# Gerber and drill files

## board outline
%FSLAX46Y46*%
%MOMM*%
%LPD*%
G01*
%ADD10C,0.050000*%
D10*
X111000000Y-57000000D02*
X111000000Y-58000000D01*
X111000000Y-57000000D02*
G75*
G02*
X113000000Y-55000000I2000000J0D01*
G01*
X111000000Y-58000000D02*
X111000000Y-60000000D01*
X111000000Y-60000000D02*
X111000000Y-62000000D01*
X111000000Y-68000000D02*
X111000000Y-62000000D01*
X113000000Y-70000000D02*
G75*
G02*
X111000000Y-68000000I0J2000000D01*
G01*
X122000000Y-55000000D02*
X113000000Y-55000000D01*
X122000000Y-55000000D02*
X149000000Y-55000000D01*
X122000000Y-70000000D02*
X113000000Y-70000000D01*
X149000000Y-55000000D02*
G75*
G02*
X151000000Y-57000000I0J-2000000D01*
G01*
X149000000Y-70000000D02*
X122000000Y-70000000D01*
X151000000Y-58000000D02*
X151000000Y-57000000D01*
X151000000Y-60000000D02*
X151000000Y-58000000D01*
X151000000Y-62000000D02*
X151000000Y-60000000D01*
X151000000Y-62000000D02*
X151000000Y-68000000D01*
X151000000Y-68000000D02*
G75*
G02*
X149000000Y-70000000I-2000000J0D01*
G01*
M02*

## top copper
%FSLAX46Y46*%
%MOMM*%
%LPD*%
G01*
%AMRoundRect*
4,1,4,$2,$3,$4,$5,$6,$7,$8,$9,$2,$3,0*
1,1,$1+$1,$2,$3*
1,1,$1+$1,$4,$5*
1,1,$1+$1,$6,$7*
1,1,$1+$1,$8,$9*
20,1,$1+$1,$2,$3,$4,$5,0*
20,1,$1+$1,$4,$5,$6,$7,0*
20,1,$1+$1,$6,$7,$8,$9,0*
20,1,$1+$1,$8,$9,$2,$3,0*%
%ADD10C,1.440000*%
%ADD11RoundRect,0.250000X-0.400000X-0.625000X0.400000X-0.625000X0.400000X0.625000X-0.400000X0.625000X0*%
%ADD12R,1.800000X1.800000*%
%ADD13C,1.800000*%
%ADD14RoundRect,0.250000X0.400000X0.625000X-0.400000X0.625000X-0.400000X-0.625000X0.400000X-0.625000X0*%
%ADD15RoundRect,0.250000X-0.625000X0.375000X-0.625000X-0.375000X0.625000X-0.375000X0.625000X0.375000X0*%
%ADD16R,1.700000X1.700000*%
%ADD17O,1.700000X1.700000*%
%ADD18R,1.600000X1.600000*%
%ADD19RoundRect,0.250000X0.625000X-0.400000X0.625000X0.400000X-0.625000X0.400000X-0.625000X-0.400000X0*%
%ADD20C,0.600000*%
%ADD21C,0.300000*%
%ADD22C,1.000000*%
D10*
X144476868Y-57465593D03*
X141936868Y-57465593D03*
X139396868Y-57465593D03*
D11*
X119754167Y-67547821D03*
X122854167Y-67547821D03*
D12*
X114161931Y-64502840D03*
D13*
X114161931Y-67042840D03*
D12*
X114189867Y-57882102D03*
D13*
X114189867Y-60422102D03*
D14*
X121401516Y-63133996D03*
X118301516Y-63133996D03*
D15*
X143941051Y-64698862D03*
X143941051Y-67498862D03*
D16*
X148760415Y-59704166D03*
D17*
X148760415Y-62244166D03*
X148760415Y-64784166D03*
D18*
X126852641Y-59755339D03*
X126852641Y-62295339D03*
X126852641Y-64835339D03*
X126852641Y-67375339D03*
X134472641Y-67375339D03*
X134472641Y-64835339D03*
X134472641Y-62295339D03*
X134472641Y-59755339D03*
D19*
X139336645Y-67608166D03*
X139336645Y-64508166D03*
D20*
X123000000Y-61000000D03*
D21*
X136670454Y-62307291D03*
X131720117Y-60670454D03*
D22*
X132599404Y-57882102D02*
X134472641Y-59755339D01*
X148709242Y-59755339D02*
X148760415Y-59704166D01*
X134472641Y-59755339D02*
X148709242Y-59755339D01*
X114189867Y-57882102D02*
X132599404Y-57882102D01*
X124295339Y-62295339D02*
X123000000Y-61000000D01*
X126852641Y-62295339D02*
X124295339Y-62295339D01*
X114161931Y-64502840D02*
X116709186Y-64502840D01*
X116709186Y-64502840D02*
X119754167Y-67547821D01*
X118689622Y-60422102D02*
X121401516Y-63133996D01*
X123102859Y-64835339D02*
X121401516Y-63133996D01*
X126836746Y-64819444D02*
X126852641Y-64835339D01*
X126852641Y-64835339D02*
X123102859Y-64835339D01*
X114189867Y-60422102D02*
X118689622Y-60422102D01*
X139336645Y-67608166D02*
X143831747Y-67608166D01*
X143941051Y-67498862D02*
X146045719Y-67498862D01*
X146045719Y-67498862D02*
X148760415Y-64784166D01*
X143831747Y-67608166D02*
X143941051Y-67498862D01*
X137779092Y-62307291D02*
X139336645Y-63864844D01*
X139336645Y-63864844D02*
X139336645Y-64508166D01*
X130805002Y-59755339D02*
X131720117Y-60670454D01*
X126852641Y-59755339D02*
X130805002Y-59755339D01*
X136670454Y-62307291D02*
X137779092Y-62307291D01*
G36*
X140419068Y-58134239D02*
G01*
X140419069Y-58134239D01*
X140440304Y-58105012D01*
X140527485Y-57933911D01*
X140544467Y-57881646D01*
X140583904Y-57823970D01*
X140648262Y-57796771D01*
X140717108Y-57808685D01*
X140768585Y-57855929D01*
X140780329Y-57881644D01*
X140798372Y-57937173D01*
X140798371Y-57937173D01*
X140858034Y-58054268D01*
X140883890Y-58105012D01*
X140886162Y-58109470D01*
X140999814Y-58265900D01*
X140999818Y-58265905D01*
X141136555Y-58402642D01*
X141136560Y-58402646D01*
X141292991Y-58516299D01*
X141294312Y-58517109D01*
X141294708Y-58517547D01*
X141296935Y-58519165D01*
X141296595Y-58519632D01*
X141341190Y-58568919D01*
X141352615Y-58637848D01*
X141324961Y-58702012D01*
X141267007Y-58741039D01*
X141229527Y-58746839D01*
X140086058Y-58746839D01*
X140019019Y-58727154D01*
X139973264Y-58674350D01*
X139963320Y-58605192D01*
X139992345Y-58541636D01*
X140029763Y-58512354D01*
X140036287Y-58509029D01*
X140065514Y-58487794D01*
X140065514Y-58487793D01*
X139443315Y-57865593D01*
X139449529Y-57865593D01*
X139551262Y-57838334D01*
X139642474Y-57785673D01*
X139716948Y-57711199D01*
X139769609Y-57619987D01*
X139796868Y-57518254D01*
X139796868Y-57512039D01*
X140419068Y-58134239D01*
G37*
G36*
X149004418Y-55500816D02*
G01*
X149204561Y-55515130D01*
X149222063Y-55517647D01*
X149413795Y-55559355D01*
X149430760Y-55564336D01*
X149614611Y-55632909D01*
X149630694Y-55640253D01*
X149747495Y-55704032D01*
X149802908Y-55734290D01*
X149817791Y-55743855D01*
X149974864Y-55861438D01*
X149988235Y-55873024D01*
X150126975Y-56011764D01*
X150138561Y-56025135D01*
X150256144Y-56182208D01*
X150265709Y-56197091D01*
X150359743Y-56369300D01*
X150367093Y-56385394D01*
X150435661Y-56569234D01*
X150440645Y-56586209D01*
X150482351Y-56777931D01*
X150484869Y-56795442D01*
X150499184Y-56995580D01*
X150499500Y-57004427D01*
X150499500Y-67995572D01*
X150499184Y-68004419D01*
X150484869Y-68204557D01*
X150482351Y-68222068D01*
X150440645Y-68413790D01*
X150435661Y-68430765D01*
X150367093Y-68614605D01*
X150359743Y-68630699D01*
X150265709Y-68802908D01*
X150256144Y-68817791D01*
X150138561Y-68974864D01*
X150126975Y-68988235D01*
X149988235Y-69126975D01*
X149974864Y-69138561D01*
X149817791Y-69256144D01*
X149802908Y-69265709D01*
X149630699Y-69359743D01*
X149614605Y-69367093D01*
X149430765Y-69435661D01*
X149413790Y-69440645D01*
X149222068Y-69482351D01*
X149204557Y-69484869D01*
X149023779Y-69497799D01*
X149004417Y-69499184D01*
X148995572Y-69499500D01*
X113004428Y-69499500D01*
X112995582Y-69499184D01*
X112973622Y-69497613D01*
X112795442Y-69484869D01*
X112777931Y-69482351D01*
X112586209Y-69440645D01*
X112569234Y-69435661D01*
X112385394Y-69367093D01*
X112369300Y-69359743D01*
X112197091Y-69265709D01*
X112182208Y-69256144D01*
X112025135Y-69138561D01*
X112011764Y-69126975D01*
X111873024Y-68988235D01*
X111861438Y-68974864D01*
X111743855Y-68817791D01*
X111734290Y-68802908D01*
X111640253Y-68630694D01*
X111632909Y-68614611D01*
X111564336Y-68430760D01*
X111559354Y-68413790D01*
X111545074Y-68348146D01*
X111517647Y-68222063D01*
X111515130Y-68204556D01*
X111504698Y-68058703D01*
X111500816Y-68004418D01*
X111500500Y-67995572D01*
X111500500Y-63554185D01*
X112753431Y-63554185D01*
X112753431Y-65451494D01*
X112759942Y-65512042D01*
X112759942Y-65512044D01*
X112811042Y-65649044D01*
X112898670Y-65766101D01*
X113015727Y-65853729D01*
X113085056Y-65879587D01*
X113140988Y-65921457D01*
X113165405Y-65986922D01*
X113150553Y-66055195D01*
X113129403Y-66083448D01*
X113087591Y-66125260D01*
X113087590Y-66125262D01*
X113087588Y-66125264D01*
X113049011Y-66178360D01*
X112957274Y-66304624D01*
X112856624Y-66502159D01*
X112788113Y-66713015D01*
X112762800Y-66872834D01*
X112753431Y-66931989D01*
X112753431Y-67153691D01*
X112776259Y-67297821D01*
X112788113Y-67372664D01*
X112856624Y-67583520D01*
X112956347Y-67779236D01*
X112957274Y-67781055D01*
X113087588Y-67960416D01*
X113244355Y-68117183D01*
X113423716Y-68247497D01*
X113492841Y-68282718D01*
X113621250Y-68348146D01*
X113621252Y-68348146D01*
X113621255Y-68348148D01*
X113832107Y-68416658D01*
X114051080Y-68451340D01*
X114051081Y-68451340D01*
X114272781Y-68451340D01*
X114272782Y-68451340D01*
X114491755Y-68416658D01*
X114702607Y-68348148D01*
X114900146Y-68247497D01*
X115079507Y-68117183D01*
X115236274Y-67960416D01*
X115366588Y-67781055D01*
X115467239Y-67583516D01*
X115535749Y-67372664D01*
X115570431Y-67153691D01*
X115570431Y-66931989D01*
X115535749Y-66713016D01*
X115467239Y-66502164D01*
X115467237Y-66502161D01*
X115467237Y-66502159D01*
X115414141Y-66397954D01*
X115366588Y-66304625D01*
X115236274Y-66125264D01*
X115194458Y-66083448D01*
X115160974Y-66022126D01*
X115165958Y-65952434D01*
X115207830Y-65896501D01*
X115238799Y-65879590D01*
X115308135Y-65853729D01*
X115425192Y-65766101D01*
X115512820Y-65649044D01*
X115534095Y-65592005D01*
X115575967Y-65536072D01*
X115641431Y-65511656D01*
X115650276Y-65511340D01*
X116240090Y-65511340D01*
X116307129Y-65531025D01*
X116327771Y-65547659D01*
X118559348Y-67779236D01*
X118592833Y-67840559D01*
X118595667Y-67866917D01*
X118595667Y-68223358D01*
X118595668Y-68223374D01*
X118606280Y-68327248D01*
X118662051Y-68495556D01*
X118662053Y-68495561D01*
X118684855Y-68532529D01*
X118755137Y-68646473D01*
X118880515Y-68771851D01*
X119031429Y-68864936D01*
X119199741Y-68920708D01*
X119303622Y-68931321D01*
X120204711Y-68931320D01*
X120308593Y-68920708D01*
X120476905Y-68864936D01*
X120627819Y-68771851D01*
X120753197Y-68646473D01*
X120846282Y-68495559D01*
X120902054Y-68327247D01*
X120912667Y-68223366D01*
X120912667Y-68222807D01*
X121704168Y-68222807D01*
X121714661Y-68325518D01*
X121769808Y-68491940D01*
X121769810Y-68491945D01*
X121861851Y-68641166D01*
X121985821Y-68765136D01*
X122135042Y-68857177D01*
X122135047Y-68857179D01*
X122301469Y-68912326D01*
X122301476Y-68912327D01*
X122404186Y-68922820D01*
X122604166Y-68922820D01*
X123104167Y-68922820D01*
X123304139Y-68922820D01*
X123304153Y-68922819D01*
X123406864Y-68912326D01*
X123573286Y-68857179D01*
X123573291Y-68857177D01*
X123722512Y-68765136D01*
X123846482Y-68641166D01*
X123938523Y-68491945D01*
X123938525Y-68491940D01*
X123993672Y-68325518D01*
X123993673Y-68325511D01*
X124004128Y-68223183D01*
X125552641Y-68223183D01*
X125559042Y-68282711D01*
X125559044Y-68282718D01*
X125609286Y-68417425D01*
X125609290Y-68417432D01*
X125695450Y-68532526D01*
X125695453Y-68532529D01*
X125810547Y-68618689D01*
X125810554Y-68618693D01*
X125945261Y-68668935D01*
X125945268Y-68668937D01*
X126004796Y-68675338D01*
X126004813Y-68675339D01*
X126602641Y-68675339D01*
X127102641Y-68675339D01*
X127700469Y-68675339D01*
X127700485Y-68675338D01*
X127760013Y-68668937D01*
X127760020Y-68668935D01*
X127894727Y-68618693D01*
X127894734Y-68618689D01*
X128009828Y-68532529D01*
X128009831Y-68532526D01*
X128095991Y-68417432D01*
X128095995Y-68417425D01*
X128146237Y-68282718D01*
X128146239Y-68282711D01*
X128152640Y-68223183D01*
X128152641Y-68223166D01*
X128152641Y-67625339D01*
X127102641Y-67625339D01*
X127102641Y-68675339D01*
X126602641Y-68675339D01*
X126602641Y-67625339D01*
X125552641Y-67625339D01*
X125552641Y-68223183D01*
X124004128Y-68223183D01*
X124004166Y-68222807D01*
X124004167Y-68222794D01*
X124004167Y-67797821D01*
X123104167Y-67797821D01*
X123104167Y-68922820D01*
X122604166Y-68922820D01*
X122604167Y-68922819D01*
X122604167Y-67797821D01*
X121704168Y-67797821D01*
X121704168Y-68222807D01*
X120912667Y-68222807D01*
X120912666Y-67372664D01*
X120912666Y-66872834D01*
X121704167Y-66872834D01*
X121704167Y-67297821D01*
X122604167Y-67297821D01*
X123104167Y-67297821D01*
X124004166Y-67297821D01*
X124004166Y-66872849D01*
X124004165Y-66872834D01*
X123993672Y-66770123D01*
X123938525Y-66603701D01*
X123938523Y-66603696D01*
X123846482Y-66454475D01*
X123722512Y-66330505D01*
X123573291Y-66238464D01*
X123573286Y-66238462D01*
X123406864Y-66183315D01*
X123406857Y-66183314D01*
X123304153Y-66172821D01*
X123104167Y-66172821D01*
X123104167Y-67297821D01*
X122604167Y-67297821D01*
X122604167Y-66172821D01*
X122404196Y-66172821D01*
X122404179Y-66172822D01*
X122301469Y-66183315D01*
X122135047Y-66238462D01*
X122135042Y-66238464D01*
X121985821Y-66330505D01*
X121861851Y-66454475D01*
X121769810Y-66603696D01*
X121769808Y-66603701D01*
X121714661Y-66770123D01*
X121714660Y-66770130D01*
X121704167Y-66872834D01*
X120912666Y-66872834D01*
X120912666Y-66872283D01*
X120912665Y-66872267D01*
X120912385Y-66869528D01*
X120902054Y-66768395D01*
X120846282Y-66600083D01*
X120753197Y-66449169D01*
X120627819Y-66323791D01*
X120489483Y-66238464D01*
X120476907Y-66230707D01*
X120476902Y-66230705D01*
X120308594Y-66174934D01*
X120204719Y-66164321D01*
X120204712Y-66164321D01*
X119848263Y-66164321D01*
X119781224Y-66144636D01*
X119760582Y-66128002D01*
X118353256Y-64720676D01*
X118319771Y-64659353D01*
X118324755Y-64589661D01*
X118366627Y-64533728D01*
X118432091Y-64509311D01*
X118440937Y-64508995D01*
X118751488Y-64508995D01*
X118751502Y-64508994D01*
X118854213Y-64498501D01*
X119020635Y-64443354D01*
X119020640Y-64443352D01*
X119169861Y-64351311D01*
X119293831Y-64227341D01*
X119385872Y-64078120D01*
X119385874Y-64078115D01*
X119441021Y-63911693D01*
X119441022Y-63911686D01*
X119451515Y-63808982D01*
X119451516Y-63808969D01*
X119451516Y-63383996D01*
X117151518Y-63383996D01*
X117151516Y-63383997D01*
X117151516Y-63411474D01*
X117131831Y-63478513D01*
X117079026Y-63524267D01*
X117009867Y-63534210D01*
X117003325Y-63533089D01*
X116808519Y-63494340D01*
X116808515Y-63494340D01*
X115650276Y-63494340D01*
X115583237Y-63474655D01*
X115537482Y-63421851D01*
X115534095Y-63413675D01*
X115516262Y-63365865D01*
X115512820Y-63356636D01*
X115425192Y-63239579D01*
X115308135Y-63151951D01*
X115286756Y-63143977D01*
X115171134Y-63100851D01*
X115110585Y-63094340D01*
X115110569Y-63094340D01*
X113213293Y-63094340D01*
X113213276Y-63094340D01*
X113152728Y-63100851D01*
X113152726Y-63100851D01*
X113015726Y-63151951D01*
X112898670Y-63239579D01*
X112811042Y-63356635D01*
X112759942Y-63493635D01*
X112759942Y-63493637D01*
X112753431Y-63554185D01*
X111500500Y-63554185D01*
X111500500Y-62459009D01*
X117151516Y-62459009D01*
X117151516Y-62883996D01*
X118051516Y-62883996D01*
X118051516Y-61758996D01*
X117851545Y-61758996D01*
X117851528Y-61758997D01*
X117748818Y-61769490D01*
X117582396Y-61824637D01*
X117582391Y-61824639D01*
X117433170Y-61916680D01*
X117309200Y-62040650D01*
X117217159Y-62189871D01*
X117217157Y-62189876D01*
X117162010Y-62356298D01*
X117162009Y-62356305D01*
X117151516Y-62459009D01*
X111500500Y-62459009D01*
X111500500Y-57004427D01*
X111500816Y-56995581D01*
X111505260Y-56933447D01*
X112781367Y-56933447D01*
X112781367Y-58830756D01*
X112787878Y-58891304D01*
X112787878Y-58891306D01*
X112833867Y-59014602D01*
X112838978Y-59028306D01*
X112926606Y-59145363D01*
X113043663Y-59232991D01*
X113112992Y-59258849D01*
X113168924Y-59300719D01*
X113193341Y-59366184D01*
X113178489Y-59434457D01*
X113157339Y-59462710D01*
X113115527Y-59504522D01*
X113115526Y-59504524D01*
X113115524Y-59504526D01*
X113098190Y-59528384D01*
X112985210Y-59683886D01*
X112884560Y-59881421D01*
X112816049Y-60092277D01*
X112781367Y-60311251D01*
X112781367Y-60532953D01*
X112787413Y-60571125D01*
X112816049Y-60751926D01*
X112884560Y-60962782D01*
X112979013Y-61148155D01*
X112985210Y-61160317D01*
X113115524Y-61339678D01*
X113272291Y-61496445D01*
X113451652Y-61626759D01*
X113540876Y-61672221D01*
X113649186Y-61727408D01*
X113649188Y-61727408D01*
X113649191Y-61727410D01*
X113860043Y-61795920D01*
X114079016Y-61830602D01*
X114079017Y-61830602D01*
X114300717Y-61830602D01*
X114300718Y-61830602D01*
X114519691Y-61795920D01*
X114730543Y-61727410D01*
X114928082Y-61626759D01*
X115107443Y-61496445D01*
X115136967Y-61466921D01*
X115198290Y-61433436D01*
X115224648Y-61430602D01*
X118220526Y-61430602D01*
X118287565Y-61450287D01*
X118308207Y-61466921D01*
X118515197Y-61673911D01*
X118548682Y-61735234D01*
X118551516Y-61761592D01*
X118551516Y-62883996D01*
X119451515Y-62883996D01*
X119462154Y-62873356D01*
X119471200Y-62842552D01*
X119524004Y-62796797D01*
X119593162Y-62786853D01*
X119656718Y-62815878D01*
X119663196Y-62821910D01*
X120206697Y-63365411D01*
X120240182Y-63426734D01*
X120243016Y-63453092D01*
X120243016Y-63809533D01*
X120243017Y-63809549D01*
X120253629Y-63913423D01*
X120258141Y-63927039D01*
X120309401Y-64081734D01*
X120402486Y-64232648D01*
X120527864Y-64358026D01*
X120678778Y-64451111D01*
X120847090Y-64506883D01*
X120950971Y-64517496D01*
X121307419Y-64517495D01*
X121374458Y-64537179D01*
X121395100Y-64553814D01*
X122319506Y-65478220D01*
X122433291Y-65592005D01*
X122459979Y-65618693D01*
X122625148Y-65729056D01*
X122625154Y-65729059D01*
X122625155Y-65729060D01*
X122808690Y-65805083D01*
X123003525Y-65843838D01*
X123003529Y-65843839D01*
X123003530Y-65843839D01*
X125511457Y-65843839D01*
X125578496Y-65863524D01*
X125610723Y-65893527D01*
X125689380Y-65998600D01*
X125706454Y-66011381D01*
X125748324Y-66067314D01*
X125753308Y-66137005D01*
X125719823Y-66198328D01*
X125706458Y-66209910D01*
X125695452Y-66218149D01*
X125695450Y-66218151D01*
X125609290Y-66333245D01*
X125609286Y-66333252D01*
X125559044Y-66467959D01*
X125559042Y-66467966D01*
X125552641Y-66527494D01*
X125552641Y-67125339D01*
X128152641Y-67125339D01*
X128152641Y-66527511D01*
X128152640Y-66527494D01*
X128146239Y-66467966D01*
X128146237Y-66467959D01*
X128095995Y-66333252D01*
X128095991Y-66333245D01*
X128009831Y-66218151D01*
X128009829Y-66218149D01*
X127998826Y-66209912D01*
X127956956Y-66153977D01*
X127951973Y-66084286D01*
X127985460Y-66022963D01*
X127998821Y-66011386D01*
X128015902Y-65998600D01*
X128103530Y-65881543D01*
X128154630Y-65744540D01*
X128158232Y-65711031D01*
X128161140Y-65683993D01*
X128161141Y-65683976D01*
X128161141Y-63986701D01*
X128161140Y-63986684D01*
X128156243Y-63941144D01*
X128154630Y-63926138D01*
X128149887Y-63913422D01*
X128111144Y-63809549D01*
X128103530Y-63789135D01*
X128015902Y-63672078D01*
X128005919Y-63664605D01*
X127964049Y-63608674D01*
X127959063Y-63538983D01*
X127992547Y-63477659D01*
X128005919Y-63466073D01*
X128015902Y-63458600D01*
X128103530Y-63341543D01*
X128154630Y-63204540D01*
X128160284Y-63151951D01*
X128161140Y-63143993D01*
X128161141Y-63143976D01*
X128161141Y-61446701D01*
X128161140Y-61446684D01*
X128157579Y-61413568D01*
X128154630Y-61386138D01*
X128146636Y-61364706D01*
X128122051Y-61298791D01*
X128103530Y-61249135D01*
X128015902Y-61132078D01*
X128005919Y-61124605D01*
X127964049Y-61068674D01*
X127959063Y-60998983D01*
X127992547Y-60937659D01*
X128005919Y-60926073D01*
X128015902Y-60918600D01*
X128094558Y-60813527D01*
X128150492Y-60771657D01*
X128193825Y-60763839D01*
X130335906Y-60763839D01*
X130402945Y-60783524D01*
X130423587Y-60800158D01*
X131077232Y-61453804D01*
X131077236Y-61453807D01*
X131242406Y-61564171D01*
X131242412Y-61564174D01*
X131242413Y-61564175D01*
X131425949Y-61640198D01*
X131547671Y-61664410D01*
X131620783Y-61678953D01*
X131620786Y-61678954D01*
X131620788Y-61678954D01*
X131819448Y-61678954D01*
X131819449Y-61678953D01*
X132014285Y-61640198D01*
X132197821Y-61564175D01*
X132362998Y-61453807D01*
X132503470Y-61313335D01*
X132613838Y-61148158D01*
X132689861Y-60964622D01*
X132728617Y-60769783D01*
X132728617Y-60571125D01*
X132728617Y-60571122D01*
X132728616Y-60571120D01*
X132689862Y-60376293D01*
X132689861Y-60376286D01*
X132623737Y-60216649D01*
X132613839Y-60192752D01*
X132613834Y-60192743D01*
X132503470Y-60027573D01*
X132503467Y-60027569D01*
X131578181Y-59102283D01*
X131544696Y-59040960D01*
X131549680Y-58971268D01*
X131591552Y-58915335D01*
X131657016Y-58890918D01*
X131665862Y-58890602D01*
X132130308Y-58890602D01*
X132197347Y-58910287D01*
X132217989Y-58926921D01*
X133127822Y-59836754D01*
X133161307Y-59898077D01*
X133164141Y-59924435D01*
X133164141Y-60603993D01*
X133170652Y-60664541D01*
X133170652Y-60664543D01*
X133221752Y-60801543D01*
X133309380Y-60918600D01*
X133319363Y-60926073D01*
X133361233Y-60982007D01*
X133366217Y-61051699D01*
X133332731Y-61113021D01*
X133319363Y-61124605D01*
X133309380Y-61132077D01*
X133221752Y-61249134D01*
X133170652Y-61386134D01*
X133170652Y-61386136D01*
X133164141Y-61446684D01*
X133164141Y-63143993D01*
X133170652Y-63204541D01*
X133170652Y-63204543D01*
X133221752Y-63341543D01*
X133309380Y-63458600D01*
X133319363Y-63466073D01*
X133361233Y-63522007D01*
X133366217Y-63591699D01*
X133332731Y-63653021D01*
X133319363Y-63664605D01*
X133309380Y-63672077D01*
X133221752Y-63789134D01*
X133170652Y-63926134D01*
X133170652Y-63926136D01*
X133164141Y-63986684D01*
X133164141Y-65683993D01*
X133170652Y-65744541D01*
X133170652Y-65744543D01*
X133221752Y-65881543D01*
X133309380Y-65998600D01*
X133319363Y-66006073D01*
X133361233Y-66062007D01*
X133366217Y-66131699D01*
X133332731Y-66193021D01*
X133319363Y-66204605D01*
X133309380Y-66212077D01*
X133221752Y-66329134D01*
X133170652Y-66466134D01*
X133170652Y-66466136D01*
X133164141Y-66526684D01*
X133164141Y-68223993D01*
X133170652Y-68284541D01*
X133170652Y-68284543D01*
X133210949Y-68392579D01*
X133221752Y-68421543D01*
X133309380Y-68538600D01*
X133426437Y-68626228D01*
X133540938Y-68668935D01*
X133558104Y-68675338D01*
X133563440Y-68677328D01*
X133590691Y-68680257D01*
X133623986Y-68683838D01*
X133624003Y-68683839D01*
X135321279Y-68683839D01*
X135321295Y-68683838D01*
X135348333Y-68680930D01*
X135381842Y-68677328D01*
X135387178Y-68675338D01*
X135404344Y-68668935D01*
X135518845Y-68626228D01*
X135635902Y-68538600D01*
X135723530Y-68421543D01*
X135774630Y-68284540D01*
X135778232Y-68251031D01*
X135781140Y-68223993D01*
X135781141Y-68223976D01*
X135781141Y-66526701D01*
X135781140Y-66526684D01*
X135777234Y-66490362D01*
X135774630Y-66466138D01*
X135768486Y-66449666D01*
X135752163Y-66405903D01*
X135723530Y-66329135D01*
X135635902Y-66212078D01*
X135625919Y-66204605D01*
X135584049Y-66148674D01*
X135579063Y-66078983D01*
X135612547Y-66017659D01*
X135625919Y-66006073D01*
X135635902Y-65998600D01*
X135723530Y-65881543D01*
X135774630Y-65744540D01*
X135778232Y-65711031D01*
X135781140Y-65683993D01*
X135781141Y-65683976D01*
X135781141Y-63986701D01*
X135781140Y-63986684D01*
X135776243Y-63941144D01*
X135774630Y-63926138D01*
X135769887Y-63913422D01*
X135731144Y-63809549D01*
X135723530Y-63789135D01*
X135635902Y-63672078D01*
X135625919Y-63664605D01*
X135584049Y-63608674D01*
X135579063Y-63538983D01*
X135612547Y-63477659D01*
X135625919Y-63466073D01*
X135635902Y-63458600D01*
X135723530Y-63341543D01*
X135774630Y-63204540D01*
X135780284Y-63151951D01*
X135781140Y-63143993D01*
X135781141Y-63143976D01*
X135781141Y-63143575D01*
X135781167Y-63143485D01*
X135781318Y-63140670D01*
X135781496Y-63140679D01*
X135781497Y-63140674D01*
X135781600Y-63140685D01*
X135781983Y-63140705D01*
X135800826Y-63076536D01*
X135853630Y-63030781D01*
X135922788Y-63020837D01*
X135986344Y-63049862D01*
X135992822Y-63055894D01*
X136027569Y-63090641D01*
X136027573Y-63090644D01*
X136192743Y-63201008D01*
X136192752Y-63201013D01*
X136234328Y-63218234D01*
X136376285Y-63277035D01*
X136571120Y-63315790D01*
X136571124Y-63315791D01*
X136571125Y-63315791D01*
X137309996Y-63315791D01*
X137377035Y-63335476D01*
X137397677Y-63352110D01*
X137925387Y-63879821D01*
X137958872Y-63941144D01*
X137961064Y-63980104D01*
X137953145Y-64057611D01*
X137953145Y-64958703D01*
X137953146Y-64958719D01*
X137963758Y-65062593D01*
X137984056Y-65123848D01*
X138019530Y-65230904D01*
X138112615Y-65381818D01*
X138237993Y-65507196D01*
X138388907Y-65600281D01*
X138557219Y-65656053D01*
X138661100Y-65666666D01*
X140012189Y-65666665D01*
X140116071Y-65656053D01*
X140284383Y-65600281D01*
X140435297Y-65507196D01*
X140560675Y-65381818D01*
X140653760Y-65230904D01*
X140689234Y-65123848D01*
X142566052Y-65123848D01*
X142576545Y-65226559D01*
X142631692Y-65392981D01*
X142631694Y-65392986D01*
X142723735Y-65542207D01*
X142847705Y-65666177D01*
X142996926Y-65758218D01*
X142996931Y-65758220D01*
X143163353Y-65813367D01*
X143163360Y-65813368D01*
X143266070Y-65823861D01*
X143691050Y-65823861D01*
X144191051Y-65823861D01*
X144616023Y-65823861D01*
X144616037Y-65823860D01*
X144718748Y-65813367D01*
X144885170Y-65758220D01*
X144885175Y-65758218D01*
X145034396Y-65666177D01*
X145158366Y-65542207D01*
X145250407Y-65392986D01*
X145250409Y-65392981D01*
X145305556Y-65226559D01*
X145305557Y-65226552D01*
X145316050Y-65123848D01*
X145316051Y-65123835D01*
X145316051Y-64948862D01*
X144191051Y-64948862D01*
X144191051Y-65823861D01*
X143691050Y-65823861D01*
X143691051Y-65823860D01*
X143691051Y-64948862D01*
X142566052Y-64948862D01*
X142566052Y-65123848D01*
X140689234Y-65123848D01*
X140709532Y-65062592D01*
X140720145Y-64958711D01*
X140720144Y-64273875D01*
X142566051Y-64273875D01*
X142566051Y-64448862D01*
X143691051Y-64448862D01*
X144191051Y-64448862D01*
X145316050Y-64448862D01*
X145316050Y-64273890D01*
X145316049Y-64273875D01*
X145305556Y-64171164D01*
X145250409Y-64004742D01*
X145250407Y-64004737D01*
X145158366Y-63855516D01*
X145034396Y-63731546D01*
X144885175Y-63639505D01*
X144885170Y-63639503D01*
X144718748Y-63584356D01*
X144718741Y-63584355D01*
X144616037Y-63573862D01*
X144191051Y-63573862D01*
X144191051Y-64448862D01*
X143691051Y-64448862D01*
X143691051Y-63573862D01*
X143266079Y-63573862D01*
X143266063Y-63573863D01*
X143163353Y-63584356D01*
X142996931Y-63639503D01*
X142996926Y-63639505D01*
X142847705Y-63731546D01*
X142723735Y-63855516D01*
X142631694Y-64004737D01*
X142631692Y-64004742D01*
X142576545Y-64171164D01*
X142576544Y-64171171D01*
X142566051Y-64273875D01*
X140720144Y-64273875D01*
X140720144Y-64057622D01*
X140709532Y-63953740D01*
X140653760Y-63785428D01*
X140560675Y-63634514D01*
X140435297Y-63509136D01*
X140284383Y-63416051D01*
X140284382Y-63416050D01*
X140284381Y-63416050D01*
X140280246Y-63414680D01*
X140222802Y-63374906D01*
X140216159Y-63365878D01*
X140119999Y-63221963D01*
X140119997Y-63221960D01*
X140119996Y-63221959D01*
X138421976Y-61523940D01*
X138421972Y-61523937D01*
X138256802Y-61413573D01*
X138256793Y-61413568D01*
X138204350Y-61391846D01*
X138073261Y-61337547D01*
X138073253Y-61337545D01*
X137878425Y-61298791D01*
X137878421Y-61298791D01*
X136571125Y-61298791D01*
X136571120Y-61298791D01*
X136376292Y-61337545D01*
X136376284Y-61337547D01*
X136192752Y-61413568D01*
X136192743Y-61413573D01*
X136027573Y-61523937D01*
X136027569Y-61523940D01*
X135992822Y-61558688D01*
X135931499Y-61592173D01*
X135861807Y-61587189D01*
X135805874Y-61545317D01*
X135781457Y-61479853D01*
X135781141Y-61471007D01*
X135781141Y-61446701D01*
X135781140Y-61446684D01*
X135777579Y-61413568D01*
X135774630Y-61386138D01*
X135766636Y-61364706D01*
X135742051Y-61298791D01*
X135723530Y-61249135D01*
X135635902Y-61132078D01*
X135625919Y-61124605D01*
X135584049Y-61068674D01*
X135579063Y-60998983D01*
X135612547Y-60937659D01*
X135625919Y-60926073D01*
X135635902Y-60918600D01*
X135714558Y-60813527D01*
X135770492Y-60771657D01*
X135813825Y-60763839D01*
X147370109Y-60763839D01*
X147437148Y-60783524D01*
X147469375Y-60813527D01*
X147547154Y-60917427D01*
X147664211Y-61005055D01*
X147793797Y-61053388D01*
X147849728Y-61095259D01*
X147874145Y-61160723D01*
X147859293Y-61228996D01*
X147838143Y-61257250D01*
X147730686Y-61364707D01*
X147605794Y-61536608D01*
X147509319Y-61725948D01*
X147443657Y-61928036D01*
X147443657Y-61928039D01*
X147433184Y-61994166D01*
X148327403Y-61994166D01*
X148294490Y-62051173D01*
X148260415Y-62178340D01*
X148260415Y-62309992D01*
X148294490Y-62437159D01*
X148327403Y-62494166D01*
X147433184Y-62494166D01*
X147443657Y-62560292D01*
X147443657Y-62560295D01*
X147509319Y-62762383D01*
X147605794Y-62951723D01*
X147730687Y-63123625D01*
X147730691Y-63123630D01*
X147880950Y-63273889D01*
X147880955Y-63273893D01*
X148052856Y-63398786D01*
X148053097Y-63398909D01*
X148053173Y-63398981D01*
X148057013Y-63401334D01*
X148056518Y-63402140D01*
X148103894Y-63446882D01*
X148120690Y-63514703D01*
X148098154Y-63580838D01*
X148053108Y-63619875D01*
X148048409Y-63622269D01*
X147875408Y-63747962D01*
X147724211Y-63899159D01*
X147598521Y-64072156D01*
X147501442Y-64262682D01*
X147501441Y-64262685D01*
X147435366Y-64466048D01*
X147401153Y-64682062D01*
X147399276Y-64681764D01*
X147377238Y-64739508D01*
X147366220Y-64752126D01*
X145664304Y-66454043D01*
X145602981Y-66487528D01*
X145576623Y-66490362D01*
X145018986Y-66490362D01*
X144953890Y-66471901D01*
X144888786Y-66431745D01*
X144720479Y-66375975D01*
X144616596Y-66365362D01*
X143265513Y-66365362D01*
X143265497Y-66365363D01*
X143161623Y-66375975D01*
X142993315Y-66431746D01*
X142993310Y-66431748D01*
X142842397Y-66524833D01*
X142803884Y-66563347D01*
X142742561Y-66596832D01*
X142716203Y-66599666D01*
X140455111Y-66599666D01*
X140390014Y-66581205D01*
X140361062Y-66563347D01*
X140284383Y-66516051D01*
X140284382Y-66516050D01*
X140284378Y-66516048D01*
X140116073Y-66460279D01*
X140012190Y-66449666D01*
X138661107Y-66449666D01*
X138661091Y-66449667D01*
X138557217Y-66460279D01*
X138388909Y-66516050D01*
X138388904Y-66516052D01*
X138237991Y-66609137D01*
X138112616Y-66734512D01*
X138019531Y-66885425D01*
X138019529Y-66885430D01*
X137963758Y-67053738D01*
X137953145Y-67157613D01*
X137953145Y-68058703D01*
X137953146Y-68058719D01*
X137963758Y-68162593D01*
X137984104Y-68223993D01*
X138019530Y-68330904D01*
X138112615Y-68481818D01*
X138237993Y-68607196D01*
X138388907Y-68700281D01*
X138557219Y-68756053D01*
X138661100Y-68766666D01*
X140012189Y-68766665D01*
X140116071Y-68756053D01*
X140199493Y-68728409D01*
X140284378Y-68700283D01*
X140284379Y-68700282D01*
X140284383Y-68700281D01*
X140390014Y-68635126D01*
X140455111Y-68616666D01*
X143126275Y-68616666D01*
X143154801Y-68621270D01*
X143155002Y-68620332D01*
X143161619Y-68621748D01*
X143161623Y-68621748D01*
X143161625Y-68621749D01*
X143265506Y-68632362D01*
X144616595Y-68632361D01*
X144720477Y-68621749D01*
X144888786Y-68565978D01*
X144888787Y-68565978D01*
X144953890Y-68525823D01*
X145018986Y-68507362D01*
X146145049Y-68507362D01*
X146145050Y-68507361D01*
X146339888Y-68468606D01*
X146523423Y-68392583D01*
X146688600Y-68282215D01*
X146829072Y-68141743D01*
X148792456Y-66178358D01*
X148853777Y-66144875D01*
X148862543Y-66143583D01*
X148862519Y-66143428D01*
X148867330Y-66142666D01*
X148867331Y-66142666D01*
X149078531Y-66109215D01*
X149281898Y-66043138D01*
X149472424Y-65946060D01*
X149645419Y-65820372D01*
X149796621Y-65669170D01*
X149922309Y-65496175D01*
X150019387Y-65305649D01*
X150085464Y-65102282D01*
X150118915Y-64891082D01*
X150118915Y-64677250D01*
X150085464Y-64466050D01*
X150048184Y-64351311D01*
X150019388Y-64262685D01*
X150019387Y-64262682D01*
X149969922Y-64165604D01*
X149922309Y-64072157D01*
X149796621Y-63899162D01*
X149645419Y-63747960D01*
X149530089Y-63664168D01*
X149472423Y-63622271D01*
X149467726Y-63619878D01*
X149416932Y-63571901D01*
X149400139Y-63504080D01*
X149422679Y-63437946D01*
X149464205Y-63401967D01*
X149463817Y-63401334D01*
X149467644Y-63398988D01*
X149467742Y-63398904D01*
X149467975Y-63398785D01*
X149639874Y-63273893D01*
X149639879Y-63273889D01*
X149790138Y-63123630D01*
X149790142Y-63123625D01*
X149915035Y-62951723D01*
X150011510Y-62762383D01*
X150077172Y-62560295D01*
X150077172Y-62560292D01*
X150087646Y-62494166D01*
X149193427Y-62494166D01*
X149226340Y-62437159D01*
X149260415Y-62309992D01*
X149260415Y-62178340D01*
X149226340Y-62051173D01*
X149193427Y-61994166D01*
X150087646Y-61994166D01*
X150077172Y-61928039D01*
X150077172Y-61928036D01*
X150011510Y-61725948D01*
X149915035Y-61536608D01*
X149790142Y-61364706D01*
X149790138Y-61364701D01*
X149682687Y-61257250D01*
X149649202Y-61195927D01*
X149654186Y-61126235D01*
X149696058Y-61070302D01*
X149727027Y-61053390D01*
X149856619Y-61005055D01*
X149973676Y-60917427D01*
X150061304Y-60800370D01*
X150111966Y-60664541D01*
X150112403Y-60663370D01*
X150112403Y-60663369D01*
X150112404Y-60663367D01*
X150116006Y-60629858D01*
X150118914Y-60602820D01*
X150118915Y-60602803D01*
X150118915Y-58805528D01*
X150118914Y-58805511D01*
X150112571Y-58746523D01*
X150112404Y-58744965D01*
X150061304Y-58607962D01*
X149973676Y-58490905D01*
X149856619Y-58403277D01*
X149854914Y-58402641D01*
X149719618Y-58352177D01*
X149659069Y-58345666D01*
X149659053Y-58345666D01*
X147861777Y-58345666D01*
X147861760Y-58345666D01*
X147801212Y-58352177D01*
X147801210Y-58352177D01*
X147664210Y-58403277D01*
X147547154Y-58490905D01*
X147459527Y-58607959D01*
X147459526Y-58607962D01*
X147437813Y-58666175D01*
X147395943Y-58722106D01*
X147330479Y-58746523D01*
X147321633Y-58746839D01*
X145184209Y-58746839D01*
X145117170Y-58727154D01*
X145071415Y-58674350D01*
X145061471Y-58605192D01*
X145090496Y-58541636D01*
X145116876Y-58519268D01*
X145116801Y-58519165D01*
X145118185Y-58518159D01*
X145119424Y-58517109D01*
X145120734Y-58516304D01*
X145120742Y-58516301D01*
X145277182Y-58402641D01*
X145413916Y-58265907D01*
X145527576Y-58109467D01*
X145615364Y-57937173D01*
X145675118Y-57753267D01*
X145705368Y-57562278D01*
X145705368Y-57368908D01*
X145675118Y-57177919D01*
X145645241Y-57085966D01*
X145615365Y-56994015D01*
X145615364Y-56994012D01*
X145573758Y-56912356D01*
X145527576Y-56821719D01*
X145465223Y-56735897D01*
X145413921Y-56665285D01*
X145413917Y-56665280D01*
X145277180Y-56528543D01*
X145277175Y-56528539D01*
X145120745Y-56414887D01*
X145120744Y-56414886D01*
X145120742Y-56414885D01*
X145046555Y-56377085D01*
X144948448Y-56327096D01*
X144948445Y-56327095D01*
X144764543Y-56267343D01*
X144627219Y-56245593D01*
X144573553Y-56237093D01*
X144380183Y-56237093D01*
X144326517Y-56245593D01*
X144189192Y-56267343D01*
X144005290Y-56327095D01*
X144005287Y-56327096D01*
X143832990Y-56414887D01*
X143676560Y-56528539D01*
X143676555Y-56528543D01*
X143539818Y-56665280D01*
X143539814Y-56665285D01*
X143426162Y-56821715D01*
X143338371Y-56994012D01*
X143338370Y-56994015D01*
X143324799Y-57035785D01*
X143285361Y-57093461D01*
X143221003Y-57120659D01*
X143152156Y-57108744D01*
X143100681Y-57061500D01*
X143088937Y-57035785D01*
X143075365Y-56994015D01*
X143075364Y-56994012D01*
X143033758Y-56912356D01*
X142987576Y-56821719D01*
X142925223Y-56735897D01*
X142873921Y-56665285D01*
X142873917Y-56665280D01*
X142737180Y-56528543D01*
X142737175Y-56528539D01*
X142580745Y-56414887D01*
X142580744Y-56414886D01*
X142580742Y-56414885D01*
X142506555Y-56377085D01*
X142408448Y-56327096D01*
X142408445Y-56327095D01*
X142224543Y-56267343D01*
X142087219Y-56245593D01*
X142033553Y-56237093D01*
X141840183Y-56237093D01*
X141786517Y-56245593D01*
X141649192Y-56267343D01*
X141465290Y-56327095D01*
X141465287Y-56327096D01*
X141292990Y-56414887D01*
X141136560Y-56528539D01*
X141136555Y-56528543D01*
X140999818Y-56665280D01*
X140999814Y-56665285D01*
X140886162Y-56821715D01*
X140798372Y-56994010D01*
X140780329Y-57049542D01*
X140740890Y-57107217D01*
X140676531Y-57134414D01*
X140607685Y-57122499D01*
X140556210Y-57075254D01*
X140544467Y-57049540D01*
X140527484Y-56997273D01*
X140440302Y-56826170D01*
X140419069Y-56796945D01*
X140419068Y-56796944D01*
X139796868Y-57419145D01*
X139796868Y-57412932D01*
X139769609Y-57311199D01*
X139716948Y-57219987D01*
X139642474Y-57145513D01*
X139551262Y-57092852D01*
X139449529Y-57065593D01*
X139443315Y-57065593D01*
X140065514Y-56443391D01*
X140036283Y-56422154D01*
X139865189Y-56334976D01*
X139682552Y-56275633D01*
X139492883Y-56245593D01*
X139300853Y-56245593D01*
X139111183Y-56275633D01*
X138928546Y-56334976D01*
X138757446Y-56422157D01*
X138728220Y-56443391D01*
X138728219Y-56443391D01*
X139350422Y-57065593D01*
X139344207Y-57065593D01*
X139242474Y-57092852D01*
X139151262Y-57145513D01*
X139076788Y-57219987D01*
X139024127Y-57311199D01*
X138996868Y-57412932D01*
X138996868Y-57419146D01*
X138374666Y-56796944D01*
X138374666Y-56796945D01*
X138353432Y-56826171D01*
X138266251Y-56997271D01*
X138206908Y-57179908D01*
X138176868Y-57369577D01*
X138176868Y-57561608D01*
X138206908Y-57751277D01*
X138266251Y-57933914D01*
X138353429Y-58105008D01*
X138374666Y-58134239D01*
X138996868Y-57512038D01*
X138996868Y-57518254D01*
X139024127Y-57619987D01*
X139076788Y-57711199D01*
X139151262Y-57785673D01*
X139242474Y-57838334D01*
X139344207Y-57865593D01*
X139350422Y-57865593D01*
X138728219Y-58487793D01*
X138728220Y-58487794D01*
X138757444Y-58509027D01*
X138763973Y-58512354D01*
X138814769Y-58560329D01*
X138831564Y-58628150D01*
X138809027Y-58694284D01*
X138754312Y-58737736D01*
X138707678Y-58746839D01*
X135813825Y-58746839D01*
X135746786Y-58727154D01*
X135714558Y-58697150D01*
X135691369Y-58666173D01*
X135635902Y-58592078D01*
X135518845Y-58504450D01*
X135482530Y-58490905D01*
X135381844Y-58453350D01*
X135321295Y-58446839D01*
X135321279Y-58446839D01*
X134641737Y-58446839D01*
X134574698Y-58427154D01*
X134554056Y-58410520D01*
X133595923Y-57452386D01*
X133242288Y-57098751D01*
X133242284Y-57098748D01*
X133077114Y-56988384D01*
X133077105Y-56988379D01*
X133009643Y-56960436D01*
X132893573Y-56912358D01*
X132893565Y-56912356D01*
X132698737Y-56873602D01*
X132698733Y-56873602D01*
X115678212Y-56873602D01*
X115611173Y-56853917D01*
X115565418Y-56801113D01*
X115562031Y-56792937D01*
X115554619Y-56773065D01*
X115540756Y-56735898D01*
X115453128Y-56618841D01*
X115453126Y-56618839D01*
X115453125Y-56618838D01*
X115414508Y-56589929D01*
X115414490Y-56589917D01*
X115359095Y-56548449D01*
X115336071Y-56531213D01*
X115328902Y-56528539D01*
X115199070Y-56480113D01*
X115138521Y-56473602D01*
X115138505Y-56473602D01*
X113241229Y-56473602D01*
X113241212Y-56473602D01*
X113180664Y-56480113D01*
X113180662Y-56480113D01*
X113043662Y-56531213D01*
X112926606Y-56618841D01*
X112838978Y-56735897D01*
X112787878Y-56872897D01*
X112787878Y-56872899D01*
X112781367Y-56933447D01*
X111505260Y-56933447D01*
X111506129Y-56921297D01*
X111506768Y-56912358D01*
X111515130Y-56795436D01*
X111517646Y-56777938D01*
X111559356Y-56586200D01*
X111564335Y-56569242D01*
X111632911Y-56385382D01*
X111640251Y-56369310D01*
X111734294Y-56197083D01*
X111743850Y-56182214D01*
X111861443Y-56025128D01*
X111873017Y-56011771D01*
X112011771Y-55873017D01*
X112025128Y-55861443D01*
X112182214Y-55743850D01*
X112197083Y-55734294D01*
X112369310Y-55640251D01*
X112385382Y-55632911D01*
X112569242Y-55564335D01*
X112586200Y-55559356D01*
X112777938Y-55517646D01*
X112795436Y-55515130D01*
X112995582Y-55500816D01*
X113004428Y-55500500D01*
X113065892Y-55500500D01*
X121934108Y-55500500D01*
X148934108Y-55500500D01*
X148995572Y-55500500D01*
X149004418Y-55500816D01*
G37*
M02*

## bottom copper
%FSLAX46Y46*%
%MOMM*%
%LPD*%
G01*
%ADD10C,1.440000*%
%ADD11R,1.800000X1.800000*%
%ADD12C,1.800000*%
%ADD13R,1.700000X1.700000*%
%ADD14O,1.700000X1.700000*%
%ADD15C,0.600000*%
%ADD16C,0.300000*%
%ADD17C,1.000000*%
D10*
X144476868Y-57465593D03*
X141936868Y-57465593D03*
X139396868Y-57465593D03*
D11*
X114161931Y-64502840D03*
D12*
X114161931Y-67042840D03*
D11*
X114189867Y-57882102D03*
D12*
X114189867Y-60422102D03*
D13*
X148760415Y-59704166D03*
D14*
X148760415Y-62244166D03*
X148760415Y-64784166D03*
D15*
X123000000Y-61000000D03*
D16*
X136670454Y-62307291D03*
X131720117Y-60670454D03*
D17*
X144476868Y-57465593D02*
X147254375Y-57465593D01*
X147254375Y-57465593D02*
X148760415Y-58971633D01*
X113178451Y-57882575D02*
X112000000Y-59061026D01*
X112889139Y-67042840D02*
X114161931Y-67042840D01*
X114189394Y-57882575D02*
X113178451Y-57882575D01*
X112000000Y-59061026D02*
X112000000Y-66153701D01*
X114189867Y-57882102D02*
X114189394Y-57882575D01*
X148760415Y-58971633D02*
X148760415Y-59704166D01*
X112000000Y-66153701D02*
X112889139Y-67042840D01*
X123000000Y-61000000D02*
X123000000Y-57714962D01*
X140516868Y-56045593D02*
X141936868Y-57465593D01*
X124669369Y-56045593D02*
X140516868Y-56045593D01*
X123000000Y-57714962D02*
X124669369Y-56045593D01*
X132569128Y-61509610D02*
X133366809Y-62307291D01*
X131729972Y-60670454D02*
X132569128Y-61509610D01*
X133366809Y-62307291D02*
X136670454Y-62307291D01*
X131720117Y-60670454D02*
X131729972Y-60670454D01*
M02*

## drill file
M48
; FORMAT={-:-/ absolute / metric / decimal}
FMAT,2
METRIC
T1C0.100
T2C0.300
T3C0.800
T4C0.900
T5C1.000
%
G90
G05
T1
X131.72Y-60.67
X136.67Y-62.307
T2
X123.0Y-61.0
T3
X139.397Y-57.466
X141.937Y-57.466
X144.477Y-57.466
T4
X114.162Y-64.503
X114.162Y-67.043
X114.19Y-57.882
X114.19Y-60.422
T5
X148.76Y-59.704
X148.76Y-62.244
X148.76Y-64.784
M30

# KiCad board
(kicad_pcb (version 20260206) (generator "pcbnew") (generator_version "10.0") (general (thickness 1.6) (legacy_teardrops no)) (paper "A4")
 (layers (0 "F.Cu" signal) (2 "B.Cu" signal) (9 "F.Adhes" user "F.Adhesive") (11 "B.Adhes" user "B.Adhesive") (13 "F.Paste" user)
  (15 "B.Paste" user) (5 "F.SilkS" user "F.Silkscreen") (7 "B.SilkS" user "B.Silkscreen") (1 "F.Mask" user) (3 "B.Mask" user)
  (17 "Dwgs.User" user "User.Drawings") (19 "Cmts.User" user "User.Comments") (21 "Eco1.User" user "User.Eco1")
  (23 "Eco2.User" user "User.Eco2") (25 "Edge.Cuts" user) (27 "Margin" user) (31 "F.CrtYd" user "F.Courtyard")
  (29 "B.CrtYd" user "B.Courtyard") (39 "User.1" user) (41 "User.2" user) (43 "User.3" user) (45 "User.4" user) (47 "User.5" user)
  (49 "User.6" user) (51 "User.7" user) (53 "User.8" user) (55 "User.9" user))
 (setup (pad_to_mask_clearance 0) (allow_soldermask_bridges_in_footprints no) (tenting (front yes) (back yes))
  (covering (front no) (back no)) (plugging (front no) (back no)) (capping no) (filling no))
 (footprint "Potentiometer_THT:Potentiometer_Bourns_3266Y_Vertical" (layer "F.Cu") (at 144.476868 57.465593)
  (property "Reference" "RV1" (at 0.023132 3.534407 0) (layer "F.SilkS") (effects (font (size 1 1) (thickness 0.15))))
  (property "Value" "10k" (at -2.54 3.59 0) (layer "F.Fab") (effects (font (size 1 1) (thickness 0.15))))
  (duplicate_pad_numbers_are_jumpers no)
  (pad "1" thru_hole circle (at 0 0) (size 1.44 1.44) (drill 0.8) (layers "*.Cu" "*.Mask") (remove_unused_layers no) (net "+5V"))
  (pad "2" thru_hole circle (at -2.54 0) (size 1.44 1.44) (drill 0.8) (layers "*.Cu" "*.Mask") (remove_unused_layers no) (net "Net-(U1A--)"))
  (pad "3" thru_hole circle (at -5.08 0) (size 1.44 1.44) (drill 0.8) (layers "*.Cu" "*.Mask") (remove_unused_layers no) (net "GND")))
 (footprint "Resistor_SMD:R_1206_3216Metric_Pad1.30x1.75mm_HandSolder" (layer "F.Cu") (at 121.304167 67.547821)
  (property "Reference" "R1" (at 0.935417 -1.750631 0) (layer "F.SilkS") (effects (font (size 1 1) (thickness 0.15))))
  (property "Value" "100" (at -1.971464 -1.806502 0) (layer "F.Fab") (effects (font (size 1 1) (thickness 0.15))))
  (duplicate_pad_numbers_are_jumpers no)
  (pad "1" smd roundrect (at -1.55 0) (size 1.3 1.75) (layers "F.Cu" "F.Mask" "F.Paste") (roundrect_rratio 0.192308) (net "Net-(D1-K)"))
  (pad "2" smd roundrect (at 1.55 0) (size 1.3 1.75) (layers "F.Cu" "F.Mask" "F.Paste") (roundrect_rratio 0.192308) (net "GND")))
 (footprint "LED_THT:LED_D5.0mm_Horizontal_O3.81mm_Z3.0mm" (layer "F.Cu") (at 114.161931 64.50284 -90)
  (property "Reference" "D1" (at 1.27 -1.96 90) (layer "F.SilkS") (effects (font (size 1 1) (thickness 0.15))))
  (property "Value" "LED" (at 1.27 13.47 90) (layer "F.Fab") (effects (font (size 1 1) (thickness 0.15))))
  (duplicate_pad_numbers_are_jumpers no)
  (pad "1" thru_hole rect (at 0 0 270) (size 1.8 1.8) (drill 0.9) (layers "*.Cu" "*.Mask") (remove_unused_layers no) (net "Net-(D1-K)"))
  (pad "2" thru_hole circle (at 2.54 0 270) (size 1.8 1.8) (drill 0.9) (layers "*.Cu" "*.Mask") (remove_unused_layers no) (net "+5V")))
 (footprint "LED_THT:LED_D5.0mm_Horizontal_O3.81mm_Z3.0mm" (layer "F.Cu") (at 114.189867 57.882102 -90)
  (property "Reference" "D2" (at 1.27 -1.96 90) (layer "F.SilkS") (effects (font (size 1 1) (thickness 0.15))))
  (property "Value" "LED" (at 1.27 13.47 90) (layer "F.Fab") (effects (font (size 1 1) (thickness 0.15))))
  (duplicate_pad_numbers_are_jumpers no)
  (pad "1" thru_hole rect (at 0 0 270) (size 1.8 1.8) (drill 0.9) (layers "*.Cu" "*.Mask") (remove_unused_layers no) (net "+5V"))
  (pad "2" thru_hole circle (at 2.54 0 270) (size 1.8 1.8) (drill 0.9) (layers "*.Cu" "*.Mask") (remove_unused_layers no) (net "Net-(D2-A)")))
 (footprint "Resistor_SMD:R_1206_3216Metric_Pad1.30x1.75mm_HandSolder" (layer "F.Cu") (at 119.851516 63.133996 180)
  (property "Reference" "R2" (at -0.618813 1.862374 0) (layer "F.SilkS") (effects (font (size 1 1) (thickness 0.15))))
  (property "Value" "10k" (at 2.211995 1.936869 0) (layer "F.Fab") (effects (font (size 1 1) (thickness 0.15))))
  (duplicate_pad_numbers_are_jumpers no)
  (pad "1" smd roundrect (at -1.55 0 180) (size 1.3 1.75) (layers "F.Cu" "F.Mask" "F.Paste") (roundrect_rratio 0.192308) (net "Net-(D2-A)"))
  (pad "2" smd roundrect (at 1.55 0 180) (size 1.3 1.75) (layers "F.Cu" "F.Mask" "F.Paste") (roundrect_rratio 0.192308) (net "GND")))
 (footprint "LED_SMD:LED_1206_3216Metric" (layer "F.Cu") (at 143.941051 66.098862 -90)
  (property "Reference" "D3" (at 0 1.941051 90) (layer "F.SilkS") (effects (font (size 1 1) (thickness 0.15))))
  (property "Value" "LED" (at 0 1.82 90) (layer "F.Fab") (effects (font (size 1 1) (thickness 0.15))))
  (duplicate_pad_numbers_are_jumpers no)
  (pad "1" smd roundrect (at -1.4 0 270) (size 1.25 1.75) (layers "F.Cu" "F.Mask" "F.Paste") (roundrect_rratio 0.2) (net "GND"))
  (pad "2" smd roundrect (at 1.4 0 270) (size 1.25 1.75) (layers "F.Cu" "F.Mask" "F.Paste") (roundrect_rratio 0.2) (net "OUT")))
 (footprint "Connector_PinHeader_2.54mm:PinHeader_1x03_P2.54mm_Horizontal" (layer "F.Cu") (at 148.760415 59.704166)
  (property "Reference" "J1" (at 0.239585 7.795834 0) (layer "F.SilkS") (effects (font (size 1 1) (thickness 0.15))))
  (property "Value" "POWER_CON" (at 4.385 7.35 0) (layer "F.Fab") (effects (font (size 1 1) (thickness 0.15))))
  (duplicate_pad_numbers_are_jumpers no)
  (pad "1" thru_hole rect (at 0 0) (size 1.7 1.7) (drill 1) (layers "*.Cu" "*.Mask") (remove_unused_layers no) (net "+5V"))
  (pad "2" thru_hole oval (at 0 2.54) (size 1.7 1.7) (drill 1) (layers "*.Cu" "*.Mask") (remove_unused_layers no) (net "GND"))
  (pad "3" thru_hole oval (at 0 5.08) (size 1.7 1.7) (drill 1) (layers "*.Cu" "*.Mask") (remove_unused_layers no) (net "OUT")))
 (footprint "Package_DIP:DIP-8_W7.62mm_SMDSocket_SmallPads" (layer "F.Cu") (at 130.662641 63.565339)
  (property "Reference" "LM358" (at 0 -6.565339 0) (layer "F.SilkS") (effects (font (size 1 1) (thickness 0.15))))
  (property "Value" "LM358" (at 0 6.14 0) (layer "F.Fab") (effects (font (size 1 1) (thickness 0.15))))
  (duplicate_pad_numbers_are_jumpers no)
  (pad "1" smd rect (at -3.81 -3.81) (size 1.6 1.6) (layers "F.Cu" "F.Mask" "F.Paste") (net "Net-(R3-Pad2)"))
  (pad "2" smd rect (at -3.81 -1.27) (size 1.6 1.6) (layers "F.Cu" "F.Mask" "F.Paste") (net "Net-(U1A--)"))
  (pad "3" smd rect (at -3.81 1.27) (size 1.6 1.6) (layers "F.Cu" "F.Mask" "F.Paste") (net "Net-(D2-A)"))
  (pad "4" smd rect (at -3.81 3.81) (size 1.6 1.6) (layers "F.Cu" "F.Mask" "F.Paste") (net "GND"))
  (pad "5" smd rect (at 3.81 3.81) (size 1.6 1.6) (layers "F.Cu" "F.Mask" "F.Paste"))
  (pad "6" smd rect (at 3.81 1.27) (size 1.6 1.6) (layers "F.Cu" "F.Mask" "F.Paste"))
  (pad "7" smd rect (at 3.81 -1.27) (size 1.6 1.6) (layers "F.Cu" "F.Mask" "F.Paste"))
  (pad "8" smd rect (at 3.81 -3.81) (size 1.6 1.6) (layers "F.Cu" "F.Mask" "F.Paste") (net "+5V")))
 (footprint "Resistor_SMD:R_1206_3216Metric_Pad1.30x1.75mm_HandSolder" (layer "F.Cu") (at 139.336645 66.058166 90)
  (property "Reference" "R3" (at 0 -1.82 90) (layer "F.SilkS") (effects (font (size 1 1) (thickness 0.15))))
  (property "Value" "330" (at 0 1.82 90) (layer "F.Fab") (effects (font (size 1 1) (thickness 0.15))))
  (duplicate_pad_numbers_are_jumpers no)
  (pad "1" smd roundrect (at -1.55 0 90) (size 1.3 1.75) (layers "F.Cu" "F.Mask" "F.Paste") (roundrect_rratio 0.192308) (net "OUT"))
  (pad "2" smd roundrect (at 1.55 0 90) (size 1.3 1.75) (layers "F.Cu" "F.Mask" "F.Paste") (roundrect_rratio 0.192308) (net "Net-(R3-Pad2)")))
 (gr_line (start 111 57) (end 111 58) (stroke (width 0.05) (type default)) (layer "Edge.Cuts"))
 (gr_arc (start 111 57) (mid 111.585786 55.585786) (end 113 55) (stroke (width 0.05) (type default)) (layer "Edge.Cuts"))
 (gr_line (start 111 58) (end 111 60) (stroke (width 0.05) (type default)) (layer "Edge.Cuts"))
 (gr_line (start 111 60) (end 111 62) (stroke (width 0.05) (type default)) (layer "Edge.Cuts"))
 (gr_line (start 111 68) (end 111 62) (stroke (width 0.05) (type default)) (layer "Edge.Cuts"))
 (gr_arc (start 113 70) (mid 111.585786 69.414214) (end 111 68) (stroke (width 0.05) (type default)) (layer "Edge.Cuts"))
 (gr_line (start 122 55) (end 113 55) (stroke (width 0.05) (type default)) (layer "Edge.Cuts"))
 (gr_line (start 122 55) (end 149 55) (stroke (width 0.05) (type default)) (layer "Edge.Cuts"))
 (gr_line (start 122 70) (end 113 70) (stroke (width 0.05) (type default)) (layer "Edge.Cuts"))
 (gr_arc (start 149 55) (mid 150.414214 55.585786) (end 151 57) (stroke (width 0.05) (type default)) (layer "Edge.Cuts"))
 (gr_line (start 149 70) (end 122 70) (stroke (width 0.05) (type default)) (layer "Edge.Cuts"))
 (gr_line (start 151 58) (end 151 57) (stroke (width 0.05) (type default)) (layer "Edge.Cuts"))
 (gr_line (start 151 60) (end 151 58) (stroke (width 0.05) (type default)) (layer "Edge.Cuts"))
 (gr_line (start 151 62) (end 151 60) (stroke (width 0.05) (type default)) (layer "Edge.Cuts"))
 (gr_line (start 151 62) (end 151 68) (stroke (width 0.05) (type default)) (layer "Edge.Cuts"))
 (gr_arc (start 151 68) (mid 150.414214 69.414214) (end 149 70) (stroke (width 0.05) (type default)) (layer "Edge.Cuts"))
 (segment (start 132.599404 57.882102) (end 134.472641 59.755339) (width 1) (layer "F.Cu") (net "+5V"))
 (segment (start 148.709242 59.755339) (end 148.760415 59.704166) (width 1) (layer "F.Cu") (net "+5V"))
 (segment (start 134.472641 59.755339) (end 148.709242 59.755339) (width 1) (layer "F.Cu") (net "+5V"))
 (segment (start 114.189867 57.882102) (end 132.599404 57.882102) (width 1) (layer "F.Cu") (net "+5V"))
 (segment (start 144.476868 57.465593) (end 147.254375 57.465593) (width 1) (layer "B.Cu") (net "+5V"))
 (segment (start 147.254375 57.465593) (end 148.760415 58.971633) (width 1) (layer "B.Cu") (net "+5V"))
 (segment (start 113.178451 57.882575) (end 112 59.061026) (width 1) (layer "B.Cu") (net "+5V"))
 (segment (start 112.889139 67.04284) (end 114.161931 67.04284) (width 1) (layer "B.Cu") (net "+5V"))
 (segment (start 114.189394 57.882575) (end 113.178451 57.882575) (width 1) (layer "B.Cu") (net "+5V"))
 (segment (start 112 59.061026) (end 112 66.153701) (width 1) (layer "B.Cu") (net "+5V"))
 (segment (start 114.189867 57.882102) (end 114.189394 57.882575) (width 1) (layer "B.Cu") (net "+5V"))
 (segment (start 148.760415 58.971633) (end 148.760415 59.704166) (width 1) (layer "B.Cu") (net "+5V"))
 (segment (start 112 66.153701) (end 112.889139 67.04284) (width 1) (layer "B.Cu") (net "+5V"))
 (segment (start 124.295339 62.295339) (end 123 61) (width 1) (layer "F.Cu") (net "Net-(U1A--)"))
 (segment (start 126.852641 62.295339) (end 124.295339 62.295339) (width 1) (layer "F.Cu") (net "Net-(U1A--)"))
 (via (at 123 61) (size 0.6) (drill 0.3) (layers "F.Cu" "B.Cu") (capping no) (covering (front no) (back no)) (plugging (front no) (back no))
  (filling no) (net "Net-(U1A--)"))
 (segment (start 123 61) (end 123 57.714962) (width 1) (layer "B.Cu") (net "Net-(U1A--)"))
 (segment (start 140.516868 56.045593) (end 141.936868 57.465593) (width 1) (layer "B.Cu") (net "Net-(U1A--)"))
 (segment (start 124.669369 56.045593) (end 140.516868 56.045593) (width 1) (layer "B.Cu") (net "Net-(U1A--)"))
 (segment (start 123 57.714962) (end 124.669369 56.045593) (width 1) (layer "B.Cu") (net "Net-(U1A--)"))
 (segment (start 114.161931 64.50284) (end 116.709186 64.50284) (width 1) (layer "F.Cu") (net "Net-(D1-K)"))
 (segment (start 116.709186 64.50284) (end 119.754167 67.547821) (width 1) (layer "F.Cu") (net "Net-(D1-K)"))
 (segment (start 118.689622 60.422102) (end 121.401516 63.133996) (width 1) (layer "F.Cu") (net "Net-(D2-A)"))
 (segment (start 123.102859 64.835339) (end 121.401516 63.133996) (width 1) (layer "F.Cu") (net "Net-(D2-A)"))
 (segment (start 126.836746 64.819444) (end 126.852641 64.835339) (width 1) (layer "F.Cu") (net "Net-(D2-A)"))
 (segment (start 126.852641 64.835339) (end 123.102859 64.835339) (width 1) (layer "F.Cu") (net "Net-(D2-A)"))
 (segment (start 114.189867 60.422102) (end 118.689622 60.422102) (width 1) (layer "F.Cu") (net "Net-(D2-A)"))
 (segment (start 139.336645 67.608166) (end 143.831747 67.608166) (width 1) (layer "F.Cu") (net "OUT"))
 (segment (start 143.941051 67.498862) (end 146.045719 67.498862) (width 1) (layer "F.Cu") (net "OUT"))
 (segment (start 146.045719 67.498862) (end 148.760415 64.784166) (width 1) (layer "F.Cu") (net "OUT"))
 (segment (start 143.831747 67.608166) (end 143.941051 67.498862) (width 1) (layer "F.Cu") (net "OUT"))
 (segment (start 137.779092 62.307291) (end 139.336645 63.864844) (width 1) (layer "F.Cu") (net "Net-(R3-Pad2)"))
 (segment (start 139.336645 63.864844) (end 139.336645 64.508166) (width 1) (layer "F.Cu") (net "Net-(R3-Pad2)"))
 (segment (start 130.805002 59.755339) (end 131.720117 60.670454) (width 1) (layer "F.Cu") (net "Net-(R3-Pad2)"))
 (segment (start 126.852641 59.755339) (end 130.805002 59.755339) (width 1) (layer "F.Cu") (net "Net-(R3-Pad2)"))
 (segment (start 136.670454 62.307291) (end 137.779092 62.307291) (width 1) (layer "F.Cu") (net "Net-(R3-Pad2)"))
 (via micro (at 136.670454 62.307291) (size 0.3) (drill 0.1) (layers "F.Cu" "B.Cu") (capping no) (covering (front no) (back no))
  (plugging (front no) (back no)) (filling no) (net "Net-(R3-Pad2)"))
 (via micro (at 131.720117 60.670454) (size 0.3) (drill 0.1) (layers "F.Cu" "B.Cu") (capping no) (covering (front no) (back no))
  (plugging (front no) (back no)) (filling no) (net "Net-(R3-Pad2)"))
 (segment (start 132.569128 61.50961) (end 133.366809 62.307291) (width 1) (layer "B.Cu") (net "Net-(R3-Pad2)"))
 (segment (start 131.729972 60.670454) (end 132.569128 61.50961) (width 1) (layer "B.Cu") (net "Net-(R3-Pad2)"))
 (segment (start 133.366809 62.307291) (end 136.670454 62.307291) (width 1) (layer "B.Cu") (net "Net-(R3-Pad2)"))
 (segment (start 131.720117 60.670454) (end 131.729972 60.670454) (width 1) (layer "B.Cu") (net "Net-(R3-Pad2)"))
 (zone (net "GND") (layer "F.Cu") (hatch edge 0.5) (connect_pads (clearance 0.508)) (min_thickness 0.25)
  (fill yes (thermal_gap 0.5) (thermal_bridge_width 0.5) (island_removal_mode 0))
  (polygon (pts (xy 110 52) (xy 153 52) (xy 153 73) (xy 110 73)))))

